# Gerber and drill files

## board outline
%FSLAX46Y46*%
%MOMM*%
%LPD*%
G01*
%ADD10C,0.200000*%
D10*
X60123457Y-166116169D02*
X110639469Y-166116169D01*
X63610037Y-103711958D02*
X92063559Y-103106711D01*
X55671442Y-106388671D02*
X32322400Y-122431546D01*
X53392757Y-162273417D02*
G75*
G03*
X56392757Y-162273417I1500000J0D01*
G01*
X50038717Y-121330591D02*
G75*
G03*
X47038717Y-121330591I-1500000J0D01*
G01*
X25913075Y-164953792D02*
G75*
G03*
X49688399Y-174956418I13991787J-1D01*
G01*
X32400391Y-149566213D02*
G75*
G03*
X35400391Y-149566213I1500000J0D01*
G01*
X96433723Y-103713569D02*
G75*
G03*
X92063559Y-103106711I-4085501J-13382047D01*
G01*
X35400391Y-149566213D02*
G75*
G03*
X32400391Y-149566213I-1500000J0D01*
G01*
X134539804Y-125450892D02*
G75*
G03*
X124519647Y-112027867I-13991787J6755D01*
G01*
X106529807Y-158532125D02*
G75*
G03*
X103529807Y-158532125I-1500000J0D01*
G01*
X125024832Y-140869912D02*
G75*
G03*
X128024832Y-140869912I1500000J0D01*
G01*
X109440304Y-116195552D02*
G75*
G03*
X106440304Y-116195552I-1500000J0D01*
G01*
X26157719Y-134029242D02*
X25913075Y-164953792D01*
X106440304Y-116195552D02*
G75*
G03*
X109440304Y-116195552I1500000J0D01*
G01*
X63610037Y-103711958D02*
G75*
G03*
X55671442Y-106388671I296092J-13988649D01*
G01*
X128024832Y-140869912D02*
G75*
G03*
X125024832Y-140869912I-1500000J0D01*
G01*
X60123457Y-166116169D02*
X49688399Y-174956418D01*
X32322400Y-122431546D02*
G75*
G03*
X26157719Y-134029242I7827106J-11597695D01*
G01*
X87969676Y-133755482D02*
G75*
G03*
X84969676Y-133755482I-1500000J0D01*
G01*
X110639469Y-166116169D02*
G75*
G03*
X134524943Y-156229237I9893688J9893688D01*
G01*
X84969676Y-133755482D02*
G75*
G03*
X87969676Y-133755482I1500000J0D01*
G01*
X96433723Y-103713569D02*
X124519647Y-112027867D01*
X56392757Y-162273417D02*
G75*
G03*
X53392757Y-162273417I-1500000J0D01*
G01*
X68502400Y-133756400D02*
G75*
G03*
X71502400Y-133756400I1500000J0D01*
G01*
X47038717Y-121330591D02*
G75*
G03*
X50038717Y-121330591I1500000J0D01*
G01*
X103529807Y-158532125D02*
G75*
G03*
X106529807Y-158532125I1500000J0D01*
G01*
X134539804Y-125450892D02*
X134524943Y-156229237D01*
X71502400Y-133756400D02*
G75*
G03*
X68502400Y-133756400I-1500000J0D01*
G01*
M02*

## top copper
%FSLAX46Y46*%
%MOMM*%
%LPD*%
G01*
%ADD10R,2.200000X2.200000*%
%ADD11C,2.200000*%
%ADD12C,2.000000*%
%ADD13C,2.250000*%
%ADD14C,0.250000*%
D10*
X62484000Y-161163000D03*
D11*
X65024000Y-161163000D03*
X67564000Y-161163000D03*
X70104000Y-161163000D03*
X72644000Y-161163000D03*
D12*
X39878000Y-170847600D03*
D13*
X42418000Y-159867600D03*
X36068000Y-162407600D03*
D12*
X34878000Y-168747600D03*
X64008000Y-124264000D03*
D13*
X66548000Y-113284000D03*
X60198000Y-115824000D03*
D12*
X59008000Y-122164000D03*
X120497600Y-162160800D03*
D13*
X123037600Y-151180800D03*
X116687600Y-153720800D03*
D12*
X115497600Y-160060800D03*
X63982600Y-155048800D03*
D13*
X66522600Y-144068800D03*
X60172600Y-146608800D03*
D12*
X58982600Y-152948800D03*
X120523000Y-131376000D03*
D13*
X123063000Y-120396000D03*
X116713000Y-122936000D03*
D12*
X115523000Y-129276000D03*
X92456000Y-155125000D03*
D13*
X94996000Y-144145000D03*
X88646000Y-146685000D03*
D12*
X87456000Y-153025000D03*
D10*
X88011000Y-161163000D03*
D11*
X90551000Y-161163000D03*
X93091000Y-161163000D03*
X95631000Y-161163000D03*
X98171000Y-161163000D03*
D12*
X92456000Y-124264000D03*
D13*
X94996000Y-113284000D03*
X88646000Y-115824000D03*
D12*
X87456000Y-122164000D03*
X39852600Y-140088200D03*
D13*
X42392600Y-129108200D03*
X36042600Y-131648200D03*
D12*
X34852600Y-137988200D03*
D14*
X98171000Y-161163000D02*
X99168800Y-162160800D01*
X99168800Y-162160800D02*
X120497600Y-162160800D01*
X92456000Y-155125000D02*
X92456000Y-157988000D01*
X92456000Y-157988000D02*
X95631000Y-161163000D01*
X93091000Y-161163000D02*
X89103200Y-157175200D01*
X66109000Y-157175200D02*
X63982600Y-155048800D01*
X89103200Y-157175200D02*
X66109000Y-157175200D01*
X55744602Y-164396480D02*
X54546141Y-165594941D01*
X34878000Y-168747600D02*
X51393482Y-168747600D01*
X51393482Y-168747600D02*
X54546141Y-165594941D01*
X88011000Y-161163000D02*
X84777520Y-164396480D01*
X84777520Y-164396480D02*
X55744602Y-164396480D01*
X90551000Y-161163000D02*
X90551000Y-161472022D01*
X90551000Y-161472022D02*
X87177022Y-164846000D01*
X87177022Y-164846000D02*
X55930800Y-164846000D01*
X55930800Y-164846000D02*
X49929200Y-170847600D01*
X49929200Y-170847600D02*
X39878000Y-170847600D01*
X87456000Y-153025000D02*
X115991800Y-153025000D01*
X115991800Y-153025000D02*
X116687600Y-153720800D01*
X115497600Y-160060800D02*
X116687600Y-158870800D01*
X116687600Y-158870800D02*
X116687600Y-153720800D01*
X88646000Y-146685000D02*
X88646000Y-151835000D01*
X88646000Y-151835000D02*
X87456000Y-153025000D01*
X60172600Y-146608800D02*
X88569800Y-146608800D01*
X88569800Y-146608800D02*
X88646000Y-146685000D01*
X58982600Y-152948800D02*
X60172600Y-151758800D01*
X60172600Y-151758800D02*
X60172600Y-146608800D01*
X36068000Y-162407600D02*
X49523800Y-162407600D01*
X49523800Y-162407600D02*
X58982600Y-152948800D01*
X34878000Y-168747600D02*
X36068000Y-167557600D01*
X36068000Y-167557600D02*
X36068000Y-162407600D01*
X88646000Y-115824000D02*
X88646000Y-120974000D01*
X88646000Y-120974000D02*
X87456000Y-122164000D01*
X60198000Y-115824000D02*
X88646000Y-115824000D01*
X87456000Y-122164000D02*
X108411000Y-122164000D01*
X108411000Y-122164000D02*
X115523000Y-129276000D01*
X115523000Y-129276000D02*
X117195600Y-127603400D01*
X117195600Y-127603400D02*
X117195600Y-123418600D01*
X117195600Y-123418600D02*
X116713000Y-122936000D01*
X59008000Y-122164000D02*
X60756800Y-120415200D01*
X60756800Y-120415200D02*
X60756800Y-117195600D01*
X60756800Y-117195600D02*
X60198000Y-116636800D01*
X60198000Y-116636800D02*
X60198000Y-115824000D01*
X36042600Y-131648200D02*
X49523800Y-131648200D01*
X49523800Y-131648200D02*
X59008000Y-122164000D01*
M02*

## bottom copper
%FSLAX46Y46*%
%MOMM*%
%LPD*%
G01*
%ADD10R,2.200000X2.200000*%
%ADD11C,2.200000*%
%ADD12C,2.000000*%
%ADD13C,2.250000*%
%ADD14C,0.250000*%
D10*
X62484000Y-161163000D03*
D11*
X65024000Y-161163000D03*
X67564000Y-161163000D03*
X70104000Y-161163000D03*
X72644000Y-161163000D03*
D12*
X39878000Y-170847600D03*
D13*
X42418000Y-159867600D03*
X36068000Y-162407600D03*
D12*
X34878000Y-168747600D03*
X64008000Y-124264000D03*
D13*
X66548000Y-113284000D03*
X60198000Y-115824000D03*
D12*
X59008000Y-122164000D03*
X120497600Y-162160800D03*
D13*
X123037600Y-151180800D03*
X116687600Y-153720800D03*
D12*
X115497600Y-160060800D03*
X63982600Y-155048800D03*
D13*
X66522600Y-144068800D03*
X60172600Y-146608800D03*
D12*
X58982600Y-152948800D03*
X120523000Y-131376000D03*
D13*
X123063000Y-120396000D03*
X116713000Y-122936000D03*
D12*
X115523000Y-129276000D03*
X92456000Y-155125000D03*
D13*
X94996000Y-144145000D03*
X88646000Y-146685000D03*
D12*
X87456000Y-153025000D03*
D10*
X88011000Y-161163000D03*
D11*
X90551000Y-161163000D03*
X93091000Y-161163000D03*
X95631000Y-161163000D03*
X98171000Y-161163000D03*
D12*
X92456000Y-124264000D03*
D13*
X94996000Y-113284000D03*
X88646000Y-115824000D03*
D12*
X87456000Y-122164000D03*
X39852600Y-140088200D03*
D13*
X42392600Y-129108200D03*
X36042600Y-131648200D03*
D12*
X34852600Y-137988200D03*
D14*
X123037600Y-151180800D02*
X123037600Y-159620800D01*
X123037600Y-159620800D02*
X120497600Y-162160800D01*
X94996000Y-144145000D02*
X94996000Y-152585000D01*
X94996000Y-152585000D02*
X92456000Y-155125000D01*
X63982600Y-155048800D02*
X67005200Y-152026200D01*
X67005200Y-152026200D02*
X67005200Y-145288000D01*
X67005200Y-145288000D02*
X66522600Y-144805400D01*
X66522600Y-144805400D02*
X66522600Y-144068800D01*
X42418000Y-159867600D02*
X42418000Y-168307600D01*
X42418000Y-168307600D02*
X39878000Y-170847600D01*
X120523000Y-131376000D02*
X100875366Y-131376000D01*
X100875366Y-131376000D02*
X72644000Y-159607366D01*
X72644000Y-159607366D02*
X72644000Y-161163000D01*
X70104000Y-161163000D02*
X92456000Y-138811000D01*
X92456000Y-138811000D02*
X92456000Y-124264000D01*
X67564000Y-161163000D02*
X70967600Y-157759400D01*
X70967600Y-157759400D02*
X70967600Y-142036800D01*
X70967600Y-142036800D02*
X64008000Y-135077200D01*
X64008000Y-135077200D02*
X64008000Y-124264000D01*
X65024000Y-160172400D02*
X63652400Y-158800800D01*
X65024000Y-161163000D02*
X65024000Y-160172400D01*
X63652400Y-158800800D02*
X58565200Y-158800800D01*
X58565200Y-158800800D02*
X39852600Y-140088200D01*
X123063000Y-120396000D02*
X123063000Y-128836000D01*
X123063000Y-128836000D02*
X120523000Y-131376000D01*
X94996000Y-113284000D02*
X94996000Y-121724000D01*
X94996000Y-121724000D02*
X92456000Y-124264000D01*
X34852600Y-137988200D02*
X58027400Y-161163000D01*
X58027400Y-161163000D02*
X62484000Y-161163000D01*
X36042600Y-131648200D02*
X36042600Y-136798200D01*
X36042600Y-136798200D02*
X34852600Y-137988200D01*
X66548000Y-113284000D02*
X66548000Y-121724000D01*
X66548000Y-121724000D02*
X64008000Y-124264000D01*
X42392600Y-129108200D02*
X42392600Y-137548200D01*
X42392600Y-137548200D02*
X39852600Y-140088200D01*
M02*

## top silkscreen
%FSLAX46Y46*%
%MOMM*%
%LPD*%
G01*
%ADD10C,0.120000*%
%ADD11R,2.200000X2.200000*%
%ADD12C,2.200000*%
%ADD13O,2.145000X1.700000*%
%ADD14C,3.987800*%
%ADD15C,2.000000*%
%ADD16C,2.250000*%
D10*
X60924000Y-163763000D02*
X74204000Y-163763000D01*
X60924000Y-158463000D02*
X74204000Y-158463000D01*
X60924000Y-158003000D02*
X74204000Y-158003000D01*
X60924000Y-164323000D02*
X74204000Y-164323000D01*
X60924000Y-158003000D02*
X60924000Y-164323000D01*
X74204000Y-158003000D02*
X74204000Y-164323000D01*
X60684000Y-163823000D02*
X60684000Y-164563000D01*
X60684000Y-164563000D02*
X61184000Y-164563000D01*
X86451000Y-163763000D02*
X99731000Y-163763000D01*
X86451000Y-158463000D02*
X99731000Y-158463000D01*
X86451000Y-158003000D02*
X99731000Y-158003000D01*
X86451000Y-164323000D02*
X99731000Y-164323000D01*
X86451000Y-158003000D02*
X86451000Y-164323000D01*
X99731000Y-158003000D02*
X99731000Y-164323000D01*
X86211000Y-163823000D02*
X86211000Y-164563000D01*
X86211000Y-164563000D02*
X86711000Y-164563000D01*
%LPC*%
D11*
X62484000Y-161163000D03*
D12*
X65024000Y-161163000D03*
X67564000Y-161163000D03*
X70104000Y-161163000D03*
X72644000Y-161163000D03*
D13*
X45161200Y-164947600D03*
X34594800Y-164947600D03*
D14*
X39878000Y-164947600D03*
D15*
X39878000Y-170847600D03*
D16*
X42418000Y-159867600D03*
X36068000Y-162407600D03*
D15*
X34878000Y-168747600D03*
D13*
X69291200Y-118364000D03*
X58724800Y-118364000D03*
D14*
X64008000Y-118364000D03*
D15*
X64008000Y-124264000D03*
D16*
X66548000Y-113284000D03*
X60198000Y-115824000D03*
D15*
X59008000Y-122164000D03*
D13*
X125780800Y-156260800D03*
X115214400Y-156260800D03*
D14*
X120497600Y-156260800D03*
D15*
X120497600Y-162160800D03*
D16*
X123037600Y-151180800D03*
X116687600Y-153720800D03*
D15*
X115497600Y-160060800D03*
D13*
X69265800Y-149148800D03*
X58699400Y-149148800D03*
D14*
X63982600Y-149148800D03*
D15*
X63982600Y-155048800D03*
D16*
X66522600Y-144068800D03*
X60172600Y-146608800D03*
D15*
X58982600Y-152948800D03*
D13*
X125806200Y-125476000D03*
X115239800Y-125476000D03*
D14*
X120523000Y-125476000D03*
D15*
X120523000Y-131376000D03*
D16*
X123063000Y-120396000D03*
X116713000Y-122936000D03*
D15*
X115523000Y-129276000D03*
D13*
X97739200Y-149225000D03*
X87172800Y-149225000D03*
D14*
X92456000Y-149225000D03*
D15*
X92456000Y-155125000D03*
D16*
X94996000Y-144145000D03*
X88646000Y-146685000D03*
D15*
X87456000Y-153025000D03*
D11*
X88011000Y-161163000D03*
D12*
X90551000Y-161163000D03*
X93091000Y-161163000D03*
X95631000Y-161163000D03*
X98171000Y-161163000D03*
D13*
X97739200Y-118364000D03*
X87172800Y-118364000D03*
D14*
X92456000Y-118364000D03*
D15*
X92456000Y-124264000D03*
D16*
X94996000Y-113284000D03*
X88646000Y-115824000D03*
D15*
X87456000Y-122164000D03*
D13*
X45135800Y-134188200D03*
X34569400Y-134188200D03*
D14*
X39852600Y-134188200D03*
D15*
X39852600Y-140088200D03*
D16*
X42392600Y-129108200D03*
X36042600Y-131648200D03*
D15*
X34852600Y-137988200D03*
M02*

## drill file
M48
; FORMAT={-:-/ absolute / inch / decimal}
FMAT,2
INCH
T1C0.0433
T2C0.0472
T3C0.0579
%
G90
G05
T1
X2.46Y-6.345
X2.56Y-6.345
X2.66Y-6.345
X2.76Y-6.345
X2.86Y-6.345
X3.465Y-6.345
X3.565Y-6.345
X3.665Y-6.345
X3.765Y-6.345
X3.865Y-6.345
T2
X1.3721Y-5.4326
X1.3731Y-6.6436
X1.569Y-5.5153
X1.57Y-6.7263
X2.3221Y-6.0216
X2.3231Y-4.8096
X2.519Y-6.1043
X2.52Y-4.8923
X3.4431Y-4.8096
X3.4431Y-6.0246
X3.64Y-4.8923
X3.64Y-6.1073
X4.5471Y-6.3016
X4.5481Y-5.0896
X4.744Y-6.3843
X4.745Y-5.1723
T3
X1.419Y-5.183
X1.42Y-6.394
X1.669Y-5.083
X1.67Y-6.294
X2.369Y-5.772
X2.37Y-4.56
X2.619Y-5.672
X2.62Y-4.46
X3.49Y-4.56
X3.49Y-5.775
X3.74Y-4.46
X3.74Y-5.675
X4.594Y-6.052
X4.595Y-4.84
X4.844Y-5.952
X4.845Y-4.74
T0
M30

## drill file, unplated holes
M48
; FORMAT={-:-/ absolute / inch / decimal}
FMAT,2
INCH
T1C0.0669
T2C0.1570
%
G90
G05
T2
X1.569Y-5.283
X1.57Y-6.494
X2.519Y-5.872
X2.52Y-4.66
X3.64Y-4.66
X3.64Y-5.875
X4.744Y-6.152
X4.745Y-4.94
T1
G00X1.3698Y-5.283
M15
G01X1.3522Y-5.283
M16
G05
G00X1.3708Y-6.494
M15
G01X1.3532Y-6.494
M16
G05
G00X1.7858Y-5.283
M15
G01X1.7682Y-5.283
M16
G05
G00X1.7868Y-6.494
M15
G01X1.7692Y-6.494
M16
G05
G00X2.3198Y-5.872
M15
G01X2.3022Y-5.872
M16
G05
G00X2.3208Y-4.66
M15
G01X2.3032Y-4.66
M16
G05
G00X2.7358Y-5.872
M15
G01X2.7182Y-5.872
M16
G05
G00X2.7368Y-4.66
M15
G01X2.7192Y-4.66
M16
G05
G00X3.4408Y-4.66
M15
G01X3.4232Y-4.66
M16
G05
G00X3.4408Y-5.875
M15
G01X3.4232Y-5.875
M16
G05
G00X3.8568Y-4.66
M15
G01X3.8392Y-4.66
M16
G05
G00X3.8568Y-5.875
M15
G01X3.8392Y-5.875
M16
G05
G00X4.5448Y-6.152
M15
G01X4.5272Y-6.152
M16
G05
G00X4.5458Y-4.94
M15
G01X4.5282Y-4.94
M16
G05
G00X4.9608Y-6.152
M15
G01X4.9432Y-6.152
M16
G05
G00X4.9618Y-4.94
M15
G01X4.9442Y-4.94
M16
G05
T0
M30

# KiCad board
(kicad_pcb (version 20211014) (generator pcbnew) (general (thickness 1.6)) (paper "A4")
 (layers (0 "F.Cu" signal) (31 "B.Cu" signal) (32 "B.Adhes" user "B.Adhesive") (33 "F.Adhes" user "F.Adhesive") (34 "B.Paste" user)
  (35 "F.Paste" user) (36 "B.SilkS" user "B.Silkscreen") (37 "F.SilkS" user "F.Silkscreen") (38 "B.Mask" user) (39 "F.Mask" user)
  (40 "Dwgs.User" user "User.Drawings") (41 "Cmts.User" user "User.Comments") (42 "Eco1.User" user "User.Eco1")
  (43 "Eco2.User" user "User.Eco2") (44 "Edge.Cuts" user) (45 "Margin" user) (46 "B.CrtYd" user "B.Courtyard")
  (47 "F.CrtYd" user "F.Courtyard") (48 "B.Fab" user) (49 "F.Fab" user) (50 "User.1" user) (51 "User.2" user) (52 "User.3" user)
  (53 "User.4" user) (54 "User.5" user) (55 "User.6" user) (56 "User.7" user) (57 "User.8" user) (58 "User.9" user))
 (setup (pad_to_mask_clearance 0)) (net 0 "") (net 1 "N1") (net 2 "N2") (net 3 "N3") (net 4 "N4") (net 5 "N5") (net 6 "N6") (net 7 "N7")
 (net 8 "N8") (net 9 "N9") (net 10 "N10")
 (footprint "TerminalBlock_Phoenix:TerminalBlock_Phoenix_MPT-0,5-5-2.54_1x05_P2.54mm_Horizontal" (layer "F.Cu") (at 62.484 161.163)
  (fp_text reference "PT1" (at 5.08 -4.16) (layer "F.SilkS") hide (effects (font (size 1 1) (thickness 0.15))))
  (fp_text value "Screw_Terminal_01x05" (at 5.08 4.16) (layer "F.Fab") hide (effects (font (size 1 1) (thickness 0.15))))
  (fp_line (start -1.56 -2.7) (end 11.72 -2.7) (layer "F.SilkS") (width 0.12))
  (fp_line (start -1.8 3.4) (end -1.3 3.4) (layer "F.SilkS") (width 0.12))
  (fp_line (start 11.72 -3.16) (end 11.72 3.16) (layer "F.SilkS") (width 0.12))
  (fp_line (start -1.8 2.66) (end -1.8 3.4) (layer "F.SilkS") (width 0.12))
  (fp_line (start -1.56 -3.16) (end -1.56 3.16) (layer "F.SilkS") (width 0.12))
  (fp_line (start -1.56 3.16) (end 11.72 3.16) (layer "F.SilkS") (width 0.12))
  (fp_line (start -1.56 -3.16) (end 11.72 -3.16) (layer "F.SilkS") (width 0.12))
  (fp_line (start -1.56 2.6) (end 11.72 2.6) (layer "F.SilkS") (width 0.12))
  (pad "1" thru_hole rect locked (at 0 0) (size 2.2 2.2) (drill 1.1) (layers *.Cu *.Mask) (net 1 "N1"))
  (pad "2" thru_hole circle locked (at 2.54 0) (size 2.2 2.2) (drill 1.1) (layers *.Cu *.Mask) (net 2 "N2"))
  (pad "3" thru_hole circle locked (at 5.08 0) (size 2.2 2.2) (drill 1.1) (layers *.Cu *.Mask) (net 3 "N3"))
  (pad "4" thru_hole circle locked (at 7.62 0) (size 2.2 2.2) (drill 1.1) (layers *.Cu *.Mask) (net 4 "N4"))
  (pad "5" thru_hole circle locked (at 10.16 0) (size 2.2 2.2) (drill 1.1) (layers *.Cu *.Mask) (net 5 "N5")))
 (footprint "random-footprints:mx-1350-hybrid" (layer "F.Cu") (at 39.878 164.9476 180)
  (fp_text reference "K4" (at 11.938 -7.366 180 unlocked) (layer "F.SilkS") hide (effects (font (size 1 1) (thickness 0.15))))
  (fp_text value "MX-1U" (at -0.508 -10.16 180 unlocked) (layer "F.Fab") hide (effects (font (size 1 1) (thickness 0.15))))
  (pad "" np_thru_hole oval (at 5.2832 0 180) (size 2.145 1.7) (drill oval 2.145 1.7) (layers F&B.Cu *.Mask))
  (pad "" np_thru_hole oval (at -5.2832 0 180) (size 2.145 1.7) (drill oval 2.145 1.7) (layers F&B.Cu *.Mask))
  (pad "" np_thru_hole circle (at 0 0) (size 3.9878 3.9878) (drill 3.9878) (layers *.Cu *.Mask))
  (pad "1" thru_hole circle (at -2.54 5.08) (size 2.25 2.25) (drill 1.47) (layers *.Cu *.Mask) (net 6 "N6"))
  (pad "1" thru_hole circle (at 0 -5.9 180) (size 2 2) (drill 1.2) (layers *.Cu *.Mask) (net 6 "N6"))
  (pad "2" thru_hole circle (at 5 -3.8 41.9) (size 2 2) (drill 1.2) (layers *.Cu *.Mask) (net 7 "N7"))
  (pad "2" thru_hole circle (at 3.81 2.54) (size 2.25 2.25) (drill 1.47) (layers *.Cu *.Mask) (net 7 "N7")))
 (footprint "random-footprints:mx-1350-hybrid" (layer "F.Cu") (at 64.008 118.364 180)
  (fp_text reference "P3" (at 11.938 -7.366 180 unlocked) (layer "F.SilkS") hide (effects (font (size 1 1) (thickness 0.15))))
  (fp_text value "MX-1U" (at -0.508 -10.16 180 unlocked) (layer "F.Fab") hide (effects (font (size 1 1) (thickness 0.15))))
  (pad "" np_thru_hole circle (at 0 0) (size 3.9878 3.9878) (drill 3.9878) (layers *.Cu *.Mask))
  (pad "" np_thru_hole oval (at -5.2832 0 180) (size 2.145 1.7) (drill oval 2.145 1.7) (layers F&B.Cu *.Mask))
  (pad "" np_thru_hole oval (at 5.2832 0 180) (size 2.145 1.7) (drill oval 2.145 1.7) (layers F&B.Cu *.Mask))
  (pad "1" thru_hole circle (at 0 -5.9 180) (size 2 2) (drill 1.2) (layers *.Cu *.Mask) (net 3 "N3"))
  (pad "1" thru_hole circle (at -2.54 5.08) (size 2.25 2.25) (drill 1.47) (layers *.Cu *.Mask) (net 3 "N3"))
  (pad "2" thru_hole circle (at 5 -3.8 41.9) (size 2 2) (drill 1.2) (layers *.Cu *.Mask) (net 1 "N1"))
  (pad "2" thru_hole circle (at 3.81 2.54) (size 2.25 2.25) (drill 1.47) (layers *.Cu *.Mask) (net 1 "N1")))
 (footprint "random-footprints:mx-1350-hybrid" (layer "F.Cu") (at 120.4976 156.2608 180)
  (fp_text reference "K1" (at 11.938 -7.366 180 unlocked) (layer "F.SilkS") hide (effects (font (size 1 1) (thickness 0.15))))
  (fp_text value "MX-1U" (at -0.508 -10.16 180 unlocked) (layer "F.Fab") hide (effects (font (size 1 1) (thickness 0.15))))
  (pad "" np_thru_hole oval (at 5.2832 0 180) (size 2.145 1.7) (drill oval 2.145 1.7) (layers F&B.Cu *.Mask))
  (pad "" np_thru_hole oval (at -5.2832 0 180) (size 2.145 1.7) (drill oval 2.145 1.7) (layers F&B.Cu *.Mask))
  (pad "" np_thru_hole circle (at 0 0) (size 3.9878 3.9878) (drill 3.9878) (layers *.Cu *.Mask))
  (pad "1" thru_hole circle (at 0 -5.9 180) (size 2 2) (drill 1.2) (layers *.Cu *.Mask) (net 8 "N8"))
  (pad "1" thru_hole circle (at -2.54 5.08) (size 2.25 2.25) (drill 1.47) (layers *.Cu *.Mask) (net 8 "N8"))
  (pad "2" thru_hole circle (at 3.81 2.54) (size 2.25 2.25) (drill 1.47) (layers *.Cu *.Mask) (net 7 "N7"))
  (pad "2" thru_hole circle (at 5 -3.8 41.9) (size 2 2) (drill 1.2) (layers *.Cu *.Mask) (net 7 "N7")))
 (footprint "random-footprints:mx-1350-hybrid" (layer "F.Cu") (at 63.9826 149.1488 180)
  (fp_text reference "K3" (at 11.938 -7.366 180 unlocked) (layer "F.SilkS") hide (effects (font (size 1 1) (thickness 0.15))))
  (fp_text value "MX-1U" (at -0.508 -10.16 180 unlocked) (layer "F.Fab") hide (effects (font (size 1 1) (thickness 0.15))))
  (pad "" np_thru_hole oval (at 5.2832 0 180) (size 2.145 1.7) (drill oval 2.145 1.7) (layers F&B.Cu *.Mask))
  (pad "" np_thru_hole oval (at -5.2832 0 180) (size 2.145 1.7) (drill oval 2.145 1.7) (layers F&B.Cu *.Mask))
  (pad "" np_thru_hole circle (at 0 0) (size 3.9878 3.9878) (drill 3.9878) (layers *.Cu *.Mask))
  (pad "1" thru_hole circle (at -2.54 5.08) (size 2.25 2.25) (drill 1.47) (layers *.Cu *.Mask) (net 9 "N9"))
  (pad "1" thru_hole circle (at 0 -5.9 180) (size 2 2) (drill 1.2) (layers *.Cu *.Mask) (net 9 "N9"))
  (pad "2" thru_hole circle (at 3.81 2.54) (size 2.25 2.25) (drill 1.47) (layers *.Cu *.Mask) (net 7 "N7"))
  (pad "2" thru_hole circle (at 5 -3.8 41.9) (size 2 2) (drill 1.2) (layers *.Cu *.Mask) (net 7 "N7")))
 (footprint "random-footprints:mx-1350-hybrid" (layer "F.Cu") (at 120.523 125.476 180)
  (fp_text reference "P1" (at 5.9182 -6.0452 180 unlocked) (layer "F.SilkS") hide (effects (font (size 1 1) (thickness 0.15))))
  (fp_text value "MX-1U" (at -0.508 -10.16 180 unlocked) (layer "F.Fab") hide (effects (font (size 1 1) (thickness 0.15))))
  (pad "" np_thru_hole oval (at 5.2832 0 180) (size 2.145 1.7) (drill oval 2.145 1.7) (layers F&B.Cu *.Mask))
  (pad "" np_thru_hole circle (at 0 0) (size 3.9878 3.9878) (drill 3.9878) (layers *.Cu *.Mask))
  (pad "" np_thru_hole oval (at -5.2832 0 180) (size 2.145 1.7) (drill oval 2.145 1.7) (layers F&B.Cu *.Mask))
  (pad "1" thru_hole circle (at -2.54 5.08) (size 2.25 2.25) (drill 1.47) (layers *.Cu *.Mask) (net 5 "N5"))
  (pad "1" thru_hole circle (at 0 -5.9 180) (size 2 2) (drill 1.2) (layers *.Cu *.Mask) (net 5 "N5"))
  (pad "2" thru_hole circle (at 5 -3.8 41.9) (size 2 2) (drill 1.2) (layers *.Cu *.Mask) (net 1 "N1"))
  (pad "2" thru_hole circle (at 3.81 2.54) (size 2.25 2.25) (drill 1.47) (layers *.Cu *.Mask) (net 1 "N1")))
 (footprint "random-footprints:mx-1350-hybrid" (layer "F.Cu") (at 92.456 149.225 180)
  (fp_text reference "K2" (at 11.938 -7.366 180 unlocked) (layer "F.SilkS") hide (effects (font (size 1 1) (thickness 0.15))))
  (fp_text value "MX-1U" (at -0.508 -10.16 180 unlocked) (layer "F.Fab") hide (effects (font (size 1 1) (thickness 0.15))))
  (pad "" np_thru_hole circle (at 0 0) (size 3.9878 3.9878) (drill 3.9878) (layers *.Cu *.Mask))
  (pad "" np_thru_hole oval (at 5.2832 0 180) (size 2.145 1.7) (drill oval 2.145 1.7) (layers F&B.Cu *.Mask))
  (pad "" np_thru_hole oval (at -5.2832 0 180) (size 2.145 1.7) (drill oval 2.145 1.7) (layers F&B.Cu *.Mask))
  (pad "1" thru_hole circle (at -2.54 5.08) (size 2.25 2.25) (drill 1.47) (layers *.Cu *.Mask) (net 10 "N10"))
  (pad "1" thru_hole circle (at 0 -5.9 180) (size 2 2) (drill 1.2) (layers *.Cu *.Mask) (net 10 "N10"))
  (pad "2" thru_hole circle (at 5 -3.8 41.9) (size 2 2) (drill 1.2) (layers *.Cu *.Mask) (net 7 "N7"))
  (pad "2" thru_hole circle (at 3.81 2.54) (size 2.25 2.25) (drill 1.47) (layers *.Cu *.Mask) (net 7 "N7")))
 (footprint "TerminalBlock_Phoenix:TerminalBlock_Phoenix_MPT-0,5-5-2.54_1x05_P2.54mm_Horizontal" (layer "F.Cu") (at 88.011 161.163)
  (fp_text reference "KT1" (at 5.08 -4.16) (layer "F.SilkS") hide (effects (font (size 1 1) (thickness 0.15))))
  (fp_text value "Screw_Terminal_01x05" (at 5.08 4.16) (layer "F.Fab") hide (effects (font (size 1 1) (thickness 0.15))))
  (fp_line (start -1.8 3.4) (end -1.3 3.4) (layer "F.SilkS") (width 0.12))
  (fp_line (start -1.56 -3.16) (end -1.56 3.16) (layer "F.SilkS") (width 0.12))
  (fp_line (start -1.56 -2.7) (end 11.72 -2.7) (layer "F.SilkS") (width 0.12))
  (fp_line (start -1.56 -3.16) (end 11.72 -3.16) (layer "F.SilkS") (width 0.12))
  (fp_line (start -1.56 3.16) (end 11.72 3.16) (layer "F.SilkS") (width 0.12))
  (fp_line (start 11.72 -3.16) (end 11.72 3.16) (layer "F.SilkS") (width 0.12))
  (fp_line (start -1.56 2.6) (end 11.72 2.6) (layer "F.SilkS") (width 0.12))
  (fp_line (start -1.8 2.66) (end -1.8 3.4) (layer "F.SilkS") (width 0.12))
  (pad "1" thru_hole rect locked (at 0 0) (size 2.2 2.2) (drill 1.1) (layers *.Cu *.Mask) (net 7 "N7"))
  (pad "2" thru_hole circle locked (at 2.54 0) (size 2.2 2.2) (drill 1.1) (layers *.Cu *.Mask) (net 6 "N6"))
  (pad "3" thru_hole circle locked (at 5.08 0) (size 2.2 2.2) (drill 1.1) (layers *.Cu *.Mask) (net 9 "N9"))
  (pad "4" thru_hole circle locked (at 7.62 0) (size 2.2 2.2) (drill 1.1) (layers *.Cu *.Mask) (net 10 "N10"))
  (pad "5" thru_hole circle locked (at 10.16 0) (size 2.2 2.2) (drill 1.1) (layers *.Cu *.Mask) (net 8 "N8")))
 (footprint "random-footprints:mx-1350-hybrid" (layer "F.Cu") (at 92.456 118.364 180)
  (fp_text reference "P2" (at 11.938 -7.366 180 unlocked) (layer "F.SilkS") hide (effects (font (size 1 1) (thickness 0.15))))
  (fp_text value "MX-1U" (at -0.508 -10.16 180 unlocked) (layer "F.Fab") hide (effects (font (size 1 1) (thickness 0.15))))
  (pad "" np_thru_hole oval (at 5.2832 0 180) (size 2.145 1.7) (drill oval 2.145 1.7) (layers F&B.Cu *.Mask))
  (pad "" np_thru_hole circle (at 0 0) (size 3.9878 3.9878) (drill 3.9878) (layers *.Cu *.Mask))
  (pad "" np_thru_hole oval (at -5.2832 0 180) (size 2.145 1.7) (drill oval 2.145 1.7) (layers F&B.Cu *.Mask))
  (pad "1" thru_hole circle (at 0 -5.9 180) (size 2 2) (drill 1.2) (layers *.Cu *.Mask) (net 4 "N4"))
  (pad "1" thru_hole circle (at -2.54 5.08) (size 2.25 2.25) (drill 1.47) (layers *.Cu *.Mask) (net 4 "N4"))
  (pad "2" thru_hole circle (at 5 -3.8 41.9) (size 2 2) (drill 1.2) (layers *.Cu *.Mask) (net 1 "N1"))
  (pad "2" thru_hole circle (at 3.81 2.54) (size 2.25 2.25) (drill 1.47) (layers *.Cu *.Mask) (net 1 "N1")))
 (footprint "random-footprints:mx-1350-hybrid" (layer "F.Cu") (at 39.8526 134.1882 180)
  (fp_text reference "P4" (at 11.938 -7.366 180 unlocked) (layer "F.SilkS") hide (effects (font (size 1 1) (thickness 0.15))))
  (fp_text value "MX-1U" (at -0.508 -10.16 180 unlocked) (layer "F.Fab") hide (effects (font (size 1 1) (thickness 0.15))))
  (pad "" np_thru_hole oval (at 5.2832 0 180) (size 2.145 1.7) (drill oval 2.145 1.7) (layers F&B.Cu *.Mask))
  (pad "" np_thru_hole circle (at 0 0) (size 3.9878 3.9878) (drill 3.9878) (layers *.Cu *.Mask))
  (pad "" np_thru_hole oval (at -5.2832 0 180) (size 2.145 1.7) (drill oval 2.145 1.7) (layers F&B.Cu *.Mask))
  (pad "1" thru_hole circle (at 0 -5.9 180) (size 2 2) (drill 1.2) (layers *.Cu *.Mask) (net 2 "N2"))
  (pad "1" thru_hole circle (at -2.54 5.08) (size 2.25 2.25) (drill 1.47) (layers *.Cu *.Mask) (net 2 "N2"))
  (pad "2" thru_hole circle (at 5 -3.8 41.9) (size 2 2) (drill 1.2) (layers *.Cu *.Mask) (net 1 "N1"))
  (pad "2" thru_hole circle (at 3.81 2.54) (size 2.25 2.25) (drill 1.47) (layers *.Cu *.Mask) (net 1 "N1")))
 (gr_line (start 60.123457 166.116169) (end 110.639469 166.116169) (layer "Edge.Cuts") (width 0.2))
 (gr_line (start 63.610037 103.711958) (end 92.063559 103.106711) (layer "Edge.Cuts") (width 0.2))
 (gr_line (start 55.671442 106.388671) (end 32.3224 122.431546) (layer "Edge.Cuts") (width 0.2))
 (gr_arc (start 56.392757 162.273417) (mid 54.892757 163.773417) (end 53.392757 162.273417) (layer "Edge.Cuts") (width 0.2))
 (gr_arc (start 47.038717 121.330591) (mid 48.538717 119.830591) (end 50.038717 121.330591) (layer "Edge.Cuts") (width 0.2))
 (gr_arc (start 49.688399 174.956418) (mid 34.478954 177.850677) (end 25.913075 164.953792) (layer "Edge.Cuts") (width 0.2))
 (gr_arc (start 35.400391 149.566213) (mid 33.900391 151.066213) (end 32.400391 149.566213) (layer "Edge.Cuts") (width 0.2))
 (gr_arc (start 92.063559 103.106711) (mid 94.272712 103.236798) (end 96.433723 103.713569) (layer "Edge.Cuts") (width 0.2))
 (gr_arc (start 32.400391 149.566213) (mid 33.900391 148.066213) (end 35.400391 149.566213) (layer "Edge.Cuts") (width 0.2))
 (gr_arc (start 124.519647 112.027867) (mid 131.760309 117.074271) (end 134.539804 125.450892) (layer "Edge.Cuts") (width 0.2))
 (gr_arc (start 103.529807 158.532125) (mid 105.029807 157.032125) (end 106.529807 158.532125) (layer "Edge.Cuts") (width 0.2))
 (gr_arc (start 128.024832 140.869912) (mid 126.524832 142.369912) (end 125.024832 140.869912) (layer "Edge.Cuts") (width 0.2))
 (gr_arc (start 106.440304 116.195552) (mid 107.940304 114.695552) (end 109.440304 116.195552) (layer "Edge.Cuts") (width 0.2))
 (gr_line (start 26.157719 134.029242) (end 25.913075 164.953792) (layer "Edge.Cuts") (width 0.2))
 (gr_arc (start 109.440304 116.195552) (mid 107.940304 117.695552) (end 106.440304 116.195552) (layer "Edge.Cuts") (width 0.2))
 (gr_arc (start 55.671442 106.388671) (mid 59.435699 104.442205) (end 63.610037 103.711958) (layer "Edge.Cuts") (width 0.2))
 (gr_arc (start 125.024832 140.869912) (mid 126.524832 139.369912) (end 128.024832 140.869912) (layer "Edge.Cuts") (width 0.2))
 (gr_line (start 60.123457 166.116169) (end 49.688399 174.956418) (layer "Edge.Cuts") (width 0.2))
 (gr_arc (start 26.157719 134.029242) (mid 27.794642 127.462092) (end 32.3224 122.431546) (layer "Edge.Cuts") (width 0.2))
 (gr_arc (start 84.969676 133.755482) (mid 86.469676 132.255482) (end 87.969676 133.755482) (layer "Edge.Cuts") (width 0.2))
 (gr_arc (start 134.524943 156.229237) (mid 125.884461 169.1505) (end 110.639469 166.116169) (layer "Edge.Cuts") (width 0.2))
 (gr_arc (start 87.969676 133.755482) (mid 86.469676 135.255482) (end 84.969676 133.755482) (layer "Edge.Cuts") (width 0.2))
 (gr_line (start 96.433723 103.713569) (end 124.519647 112.027867) (layer "Edge.Cuts") (width 0.2))
 (gr_arc (start 53.392757 162.273417) (mid 54.892757 160.773417) (end 56.392757 162.273417) (layer "Edge.Cuts") (width 0.2))
 (gr_arc (start 71.5024 133.7564) (mid 70.0024 135.2564) (end 68.5024 133.7564) (layer "Edge.Cuts") (width 0.2))
 (gr_arc (start 50.038717 121.330591) (mid 48.538717 122.830591) (end 47.038717 121.330591) (layer "Edge.Cuts") (width 0.2))
 (gr_arc (start 106.529807 158.532125) (mid 105.029807 160.032125) (end 103.529807 158.532125) (layer "Edge.Cuts") (width 0.2))
 (gr_line (start 134.539804 125.450892) (end 134.524943 156.229237) (layer "Edge.Cuts") (width 0.2))
 (gr_arc (start 68.5024 133.7564) (mid 70.0024 132.2564) (end 71.5024 133.7564) (layer "Edge.Cuts") (width 0.2))
 (segment (start 98.171 161.163) (end 99.1688 162.1608) (width 0.25) (layer "F.Cu") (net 8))
 (segment (start 99.1688 162.1608) (end 120.4976 162.1608) (width 0.25) (layer "F.Cu") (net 8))
 (segment (start 123.0376 151.1808) (end 123.0376 159.6208) (width 0.25) (layer "B.Cu") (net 8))
 (segment (start 123.0376 159.6208) (end 120.4976 162.1608) (width 0.25) (layer "B.Cu") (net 8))
 (segment (start 115.4976 160.0608) (end 116.6876 158.8708) (width 0.25) (layer "F.Cu") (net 7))
 (segment (start 88.646 146.685) (end 88.646 151.835) (width 0.25) (layer "F.Cu") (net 7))
 (segment (start 87.456 153.025) (end 115.9918 153.025) (width 0.25) (layer "F.Cu") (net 7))
 (segment (start 88.011 161.163) (end 84.77752 164.39648) (width 0.25) (layer "F.Cu") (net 7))
 (segment (start 116.6876 158.8708) (end 116.6876 153.7208) (width 0.25) (layer "F.Cu") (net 7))
 (segment (start 88.646 151.835) (end 87.456 153.025) (width 0.25) (layer "F.Cu") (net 7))
 (segment (start 34.878 168.7476) (end 51.393482 168.7476) (width 0.25) (layer "F.Cu") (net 7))
 (segment (start 49.5238 162.4076) (end 58.9826 152.9488) (width 0.25) (layer "F.Cu") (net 7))
 (segment (start 84.77752 164.39648) (end 55.744602 164.39648) (width 0.25) (layer "F.Cu") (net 7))
 (segment (start 36.068 167.5576) (end 36.068 162.4076) (width 0.25) (layer "F.Cu") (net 7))
 (segment (start 88.5698 146.6088) (end 88.646 146.685) (width 0.25) (layer "F.Cu") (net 7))
 (segment (start 58.9826 152.9488) (end 60.1726 151.7588) (width 0.25) (layer "F.Cu") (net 7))
 (segment (start 115.9918 153.025) (end 116.6876 153.7208) (width 0.25) (layer "F.Cu") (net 7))
 (segment (start 36.068 162.4076) (end 49.5238 162.4076) (width 0.25) (layer "F.Cu") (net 7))
 (segment (start 60.1726 146.6088) (end 88.5698 146.6088) (width 0.25) (layer "F.Cu") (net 7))
 (segment (start 34.878 168.7476) (end 36.068 167.5576) (width 0.25) (layer "F.Cu") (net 7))
 (segment (start 60.1726 151.7588) (end 60.1726 146.6088) (width 0.25) (layer "F.Cu") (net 7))
 (segment (start 51.393482 168.7476) (end 54.546141 165.594941) (width 0.25) (layer "F.Cu") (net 7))
 (segment (start 55.744602 164.39648) (end 54.546141 165.594941) (width 0.25) (layer "F.Cu") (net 7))
 (segment (start 123.063 120.396) (end 123.063 128.836) (width 0.25) (layer "B.Cu") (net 5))
 (segment (start 123.063 128.836) (end 120.523 131.376) (width 0.25) (layer "B.Cu") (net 5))
 (segment (start 120.523 131.376) (end 100.875366 131.376) (width 0.25) (layer "B.Cu") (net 5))
 (segment (start 100.875366 131.376) (end 72.644 159.607366) (width 0.25) (layer "B.Cu") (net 5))
 (segment (start 72.644 159.607366) (end 72.644 161.163) (width 0.25) (layer "B.Cu") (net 5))
 (segment (start 70.9676 142.0368) (end 64.008 135.0772) (width 0.25) (layer "B.Cu") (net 3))
 (segment (start 66.548 121.724) (end 64.008 124.264) (width 0.25) (layer "B.Cu") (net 3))
 (segment (start 64.008 135.0772) (end 64.008 124.264) (width 0.25) (layer "B.Cu") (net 3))
 (segment (start 66.548 113.284) (end 66.548 121.724) (width 0.25) (layer "B.Cu") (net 3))
 (segment (start 70.9676 157.7594) (end 70.9676 142.0368) (width 0.25) (layer "B.Cu") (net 3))
 (segment (start 67.564 161.163) (end 70.9676 157.7594) (width 0.25) (layer "B.Cu") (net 3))
 (segment (start 92.456 157.988) (end 95.631 161.163) (width 0.25) (layer "F.Cu") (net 10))
 (segment (start 92.456 155.125) (end 92.456 157.988) (width 0.25) (layer "F.Cu") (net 10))
 (segment (start 94.996 144.145) (end 94.996 152.585) (width 0.25) (layer "B.Cu") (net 10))
 (segment (start 94.996 152.585) (end 92.456 155.125) (width 0.25) (layer "B.Cu") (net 10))
 (segment (start 93.091 161.163) (end 89.1032 157.1752) (width 0.25) (layer "F.Cu") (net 9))
 (segment (start 66.109 157.1752) (end 63.9826 155.0488) (width 0.25) (layer "F.Cu") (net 9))
 (segment (start 89.1032 157.1752) (end 66.109 157.1752) (width 0.25) (layer "F.Cu") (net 9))
 (segment (start 67.0052 145.288) (end 66.5226 144.8054) (width 0.25) (layer "B.Cu") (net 9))
 (segment (start 63.9826 155.0488) (end 67.0052 152.0262) (width 0.25) (layer "B.Cu") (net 9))
 (segment (start 66.5226 144.8054) (end 66.5226 144.0688) (width 0.25) (layer "B.Cu") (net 9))
 (segment (start 67.0052 152.0262) (end 67.0052 145.288) (width 0.25) (layer "B.Cu") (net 9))
 (segment (start 90.551 161.472022) (end 87.177022 164.846) (width 0.25) (layer "F.Cu") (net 6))
 (segment (start 90.551 161.163) (end 90.551 161.472022) (width 0.25) (layer "F.Cu") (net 6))
 (segment (start 55.9308 164.846) (end 49.9292 170.8476) (width 0.25) (layer "F.Cu") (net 6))
 (segment (start 49.9292 170.8476) (end 39.878 170.8476) (width 0.25) (layer "F.Cu") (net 6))
 (segment (start 87.177022 164.846) (end 55.9308 164.846) (width 0.25) (layer "F.Cu") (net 6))
 (segment (start 42.418 168.3076) (end 39.878 170.8476) (width 0.25) (layer "B.Cu") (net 6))
 (segment (start 42.418 159.8676) (end 42.418 168.3076) (width 0.25) (layer "B.Cu") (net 6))
 (segment (start 108.411 122.164) (end 115.523 129.276) (width 0.25) (layer "F.Cu") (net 1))
 (segment (start 60.198 115.824) (end 88.646 115.824) (width 0.25) (layer "F.Cu") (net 1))
 (segment (start 87.456 122.164) (end 108.411 122.164) (width 0.25) (layer "F.Cu") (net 1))
 (segment (start 49.5238 131.6482) (end 59.008 122.164) (width 0.25) (layer "F.Cu") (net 1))
 (segment (start 117.1956 127.6034) (end 117.1956 123.4186) (width 0.25) (layer "F.Cu") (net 1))
 (segment (start 36.0426 131.6482) (end 49.5238 131.6482) (width 0.25) (layer "F.Cu") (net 1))
 (segment (start 60.198 116.6368) (end 60.198 115.824) (width 0.25) (layer "F.Cu") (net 1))
 (segment (start 60.7568 117.1956) (end 60.198 116.6368) (width 0.25) (layer "F.Cu") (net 1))
 (segment (start 117.1956 123.4186) (end 116.713 122.936) (width 0.25) (layer "F.Cu") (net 1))
 (segment (start 88.646 120.974) (end 87.456 122.164) (width 0.25) (layer "F.Cu") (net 1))
 (segment (start 59.008 122.164) (end 60.7568 120.4152) (width 0.25) (layer "F.Cu") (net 1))
 (segment (start 115.523 129.276) (end 117.1956 127.6034) (width 0.25) (layer "F.Cu") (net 1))
 (segment (start 60.7568 120.4152) (end 60.7568 117.1956) (width 0.25) (layer "F.Cu") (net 1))
 (segment (start 88.646 115.824) (end 88.646 120.974) (width 0.25) (layer "F.Cu") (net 1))
 (segment (start 58.0274 161.163) (end 62.484 161.163) (width 0.25) (layer "B.Cu") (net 1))
 (segment (start 36.0426 136.7982) (end 34.8526 137.9882) (width 0.25) (layer "B.Cu") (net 1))
 (segment (start 34.8526 137.9882) (end 58.0274 161.163) (width 0.25) (layer "B.Cu") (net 1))
 (segment (start 36.0426 131.6482) (end 36.0426 136.7982) (width 0.25) (layer "B.Cu") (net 1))
 (segment (start 92.456 138.811) (end 92.456 124.264) (width 0.25) (layer "B.Cu") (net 4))
 (segment (start 94.996 121.724) (end 92.456 124.264) (width 0.25) (layer "B.Cu") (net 4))
 (segment (start 94.996 113.284) (end 94.996 121.724) (width 0.25) (layer "B.Cu") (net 4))
 (segment (start 70.104 161.163) (end 92.456 138.811) (width 0.25) (layer "B.Cu") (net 4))
 (segment (start 65.024 161.163) (end 65.024 160.1724) (width 0.25) (layer "B.Cu") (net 2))
 (segment (start 42.3926 137.5482) (end 39.8526 140.0882) (width 0.25) (layer "B.Cu") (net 2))
 (segment (start 42.3926 129.1082) (end 42.3926 137.5482) (width 0.25) (layer "B.Cu") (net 2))
 (segment (start 58.5652 158.8008) (end 39.8526 140.0882) (width 0.25) (layer "B.Cu") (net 2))
 (segment (start 63.6524 158.8008) (end 58.5652 158.8008) (width 0.25) (layer "B.Cu") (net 2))
 (segment (start 65.024 160.1724) (end 63.6524 158.8008) (width 0.25) (layer "B.Cu") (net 2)))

